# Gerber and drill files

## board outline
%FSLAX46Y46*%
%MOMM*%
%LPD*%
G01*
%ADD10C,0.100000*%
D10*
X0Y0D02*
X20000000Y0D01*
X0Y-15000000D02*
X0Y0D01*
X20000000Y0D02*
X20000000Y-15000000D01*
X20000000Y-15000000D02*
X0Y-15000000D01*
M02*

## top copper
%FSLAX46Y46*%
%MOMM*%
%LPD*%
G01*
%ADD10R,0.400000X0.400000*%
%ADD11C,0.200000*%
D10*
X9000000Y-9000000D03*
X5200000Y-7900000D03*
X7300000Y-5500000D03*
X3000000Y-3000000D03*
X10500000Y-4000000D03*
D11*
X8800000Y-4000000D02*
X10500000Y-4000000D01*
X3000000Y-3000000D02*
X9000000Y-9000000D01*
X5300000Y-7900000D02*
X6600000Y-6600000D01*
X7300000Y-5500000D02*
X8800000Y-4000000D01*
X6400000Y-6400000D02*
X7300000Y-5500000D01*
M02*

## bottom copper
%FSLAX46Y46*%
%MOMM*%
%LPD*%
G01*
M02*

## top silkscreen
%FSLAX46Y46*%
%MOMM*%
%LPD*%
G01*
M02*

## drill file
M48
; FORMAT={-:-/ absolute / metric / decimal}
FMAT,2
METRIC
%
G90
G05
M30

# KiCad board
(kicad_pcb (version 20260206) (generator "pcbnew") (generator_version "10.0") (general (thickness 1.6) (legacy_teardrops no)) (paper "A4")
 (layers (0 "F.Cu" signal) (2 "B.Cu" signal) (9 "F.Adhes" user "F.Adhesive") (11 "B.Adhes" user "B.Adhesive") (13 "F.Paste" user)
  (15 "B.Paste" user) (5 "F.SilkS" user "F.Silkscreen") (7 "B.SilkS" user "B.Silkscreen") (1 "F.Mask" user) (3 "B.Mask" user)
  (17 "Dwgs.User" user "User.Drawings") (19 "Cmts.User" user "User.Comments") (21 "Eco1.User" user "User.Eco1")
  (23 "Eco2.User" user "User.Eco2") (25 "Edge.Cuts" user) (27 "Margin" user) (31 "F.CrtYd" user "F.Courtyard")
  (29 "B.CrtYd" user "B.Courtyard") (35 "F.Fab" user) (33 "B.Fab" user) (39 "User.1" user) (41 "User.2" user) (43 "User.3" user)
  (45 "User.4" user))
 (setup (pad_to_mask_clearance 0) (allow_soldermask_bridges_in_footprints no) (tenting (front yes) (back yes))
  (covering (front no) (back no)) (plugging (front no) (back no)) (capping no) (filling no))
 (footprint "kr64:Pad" (layer "F.Cu") (at 9 9)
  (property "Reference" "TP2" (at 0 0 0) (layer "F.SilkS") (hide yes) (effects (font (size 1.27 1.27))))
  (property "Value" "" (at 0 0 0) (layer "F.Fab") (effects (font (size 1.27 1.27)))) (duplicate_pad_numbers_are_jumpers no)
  (pad "1" smd rect (at 0 0) (size 0.4 0.4) (layers "F.Cu" "F.Mask" "F.Paste") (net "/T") (thermal_bridge_angle 45)))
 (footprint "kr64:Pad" (layer "F.Cu") (at 5.2 7.9)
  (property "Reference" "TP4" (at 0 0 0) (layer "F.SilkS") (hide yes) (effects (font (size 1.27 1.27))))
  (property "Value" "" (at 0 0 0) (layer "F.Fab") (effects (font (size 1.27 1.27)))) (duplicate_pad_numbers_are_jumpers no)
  (pad "1" smd rect (at 0 0) (size 0.4 0.4) (layers "F.Cu" "F.Mask" "F.Paste") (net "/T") (thermal_bridge_angle 45)))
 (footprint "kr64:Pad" (layer "F.Cu") (at 7.3 5.5)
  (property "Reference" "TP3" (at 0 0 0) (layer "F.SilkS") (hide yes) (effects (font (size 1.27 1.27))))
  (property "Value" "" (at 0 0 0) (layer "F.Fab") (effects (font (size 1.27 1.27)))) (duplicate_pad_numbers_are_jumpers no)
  (pad "1" smd rect (at 0 0) (size 0.4 0.4) (layers "F.Cu" "F.Mask" "F.Paste") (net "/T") (thermal_bridge_angle 45)))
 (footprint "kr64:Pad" (layer "F.Cu") (at 3 3)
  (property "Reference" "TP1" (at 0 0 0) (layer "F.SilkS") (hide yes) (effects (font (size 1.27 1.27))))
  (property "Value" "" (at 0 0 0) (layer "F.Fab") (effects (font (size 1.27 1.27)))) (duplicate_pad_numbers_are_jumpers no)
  (pad "1" smd rect (at 0 0) (size 0.4 0.4) (layers "F.Cu" "F.Mask" "F.Paste") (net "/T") (thermal_bridge_angle 45)))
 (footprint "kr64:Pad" (layer "F.Cu") (at 10.5 4)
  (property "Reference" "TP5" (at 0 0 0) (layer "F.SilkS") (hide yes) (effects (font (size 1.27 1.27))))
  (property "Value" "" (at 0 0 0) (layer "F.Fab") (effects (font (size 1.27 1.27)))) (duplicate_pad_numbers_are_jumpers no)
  (pad "1" smd rect (at 0 0) (size 0.4 0.4) (layers "F.Cu" "F.Mask" "F.Paste") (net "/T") (thermal_bridge_angle 45)))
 (gr_line (start 0 0) (end 20 0) (stroke (width 0.1) (type default)) (layer "Edge.Cuts"))
 (gr_line (start 0 15) (end 0 0) (stroke (width 0.1) (type default)) (layer "Edge.Cuts"))
 (gr_line (start 20 0) (end 20 15) (stroke (width 0.1) (type default)) (layer "Edge.Cuts"))
 (gr_line (start 20 15) (end 0 15) (stroke (width 0.1) (type default)) (layer "Edge.Cuts"))
 (segment (start 8.8 4) (end 10.5 4) (width 0.2) (layer "F.Cu") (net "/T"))
 (segment (start 3 3) (end 9 9) (width 0.2) (layer "F.Cu") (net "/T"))
 (segment (start 5.3 7.9) (end 6.6 6.6) (width 0.2) (layer "F.Cu") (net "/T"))
 (segment (start 7.3 5.5) (end 8.8 4) (width 0.2) (layer "F.Cu") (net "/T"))
 (segment (start 6.4 6.4) (end 7.3 5.5) (width 0.2) (layer "F.Cu") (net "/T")))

